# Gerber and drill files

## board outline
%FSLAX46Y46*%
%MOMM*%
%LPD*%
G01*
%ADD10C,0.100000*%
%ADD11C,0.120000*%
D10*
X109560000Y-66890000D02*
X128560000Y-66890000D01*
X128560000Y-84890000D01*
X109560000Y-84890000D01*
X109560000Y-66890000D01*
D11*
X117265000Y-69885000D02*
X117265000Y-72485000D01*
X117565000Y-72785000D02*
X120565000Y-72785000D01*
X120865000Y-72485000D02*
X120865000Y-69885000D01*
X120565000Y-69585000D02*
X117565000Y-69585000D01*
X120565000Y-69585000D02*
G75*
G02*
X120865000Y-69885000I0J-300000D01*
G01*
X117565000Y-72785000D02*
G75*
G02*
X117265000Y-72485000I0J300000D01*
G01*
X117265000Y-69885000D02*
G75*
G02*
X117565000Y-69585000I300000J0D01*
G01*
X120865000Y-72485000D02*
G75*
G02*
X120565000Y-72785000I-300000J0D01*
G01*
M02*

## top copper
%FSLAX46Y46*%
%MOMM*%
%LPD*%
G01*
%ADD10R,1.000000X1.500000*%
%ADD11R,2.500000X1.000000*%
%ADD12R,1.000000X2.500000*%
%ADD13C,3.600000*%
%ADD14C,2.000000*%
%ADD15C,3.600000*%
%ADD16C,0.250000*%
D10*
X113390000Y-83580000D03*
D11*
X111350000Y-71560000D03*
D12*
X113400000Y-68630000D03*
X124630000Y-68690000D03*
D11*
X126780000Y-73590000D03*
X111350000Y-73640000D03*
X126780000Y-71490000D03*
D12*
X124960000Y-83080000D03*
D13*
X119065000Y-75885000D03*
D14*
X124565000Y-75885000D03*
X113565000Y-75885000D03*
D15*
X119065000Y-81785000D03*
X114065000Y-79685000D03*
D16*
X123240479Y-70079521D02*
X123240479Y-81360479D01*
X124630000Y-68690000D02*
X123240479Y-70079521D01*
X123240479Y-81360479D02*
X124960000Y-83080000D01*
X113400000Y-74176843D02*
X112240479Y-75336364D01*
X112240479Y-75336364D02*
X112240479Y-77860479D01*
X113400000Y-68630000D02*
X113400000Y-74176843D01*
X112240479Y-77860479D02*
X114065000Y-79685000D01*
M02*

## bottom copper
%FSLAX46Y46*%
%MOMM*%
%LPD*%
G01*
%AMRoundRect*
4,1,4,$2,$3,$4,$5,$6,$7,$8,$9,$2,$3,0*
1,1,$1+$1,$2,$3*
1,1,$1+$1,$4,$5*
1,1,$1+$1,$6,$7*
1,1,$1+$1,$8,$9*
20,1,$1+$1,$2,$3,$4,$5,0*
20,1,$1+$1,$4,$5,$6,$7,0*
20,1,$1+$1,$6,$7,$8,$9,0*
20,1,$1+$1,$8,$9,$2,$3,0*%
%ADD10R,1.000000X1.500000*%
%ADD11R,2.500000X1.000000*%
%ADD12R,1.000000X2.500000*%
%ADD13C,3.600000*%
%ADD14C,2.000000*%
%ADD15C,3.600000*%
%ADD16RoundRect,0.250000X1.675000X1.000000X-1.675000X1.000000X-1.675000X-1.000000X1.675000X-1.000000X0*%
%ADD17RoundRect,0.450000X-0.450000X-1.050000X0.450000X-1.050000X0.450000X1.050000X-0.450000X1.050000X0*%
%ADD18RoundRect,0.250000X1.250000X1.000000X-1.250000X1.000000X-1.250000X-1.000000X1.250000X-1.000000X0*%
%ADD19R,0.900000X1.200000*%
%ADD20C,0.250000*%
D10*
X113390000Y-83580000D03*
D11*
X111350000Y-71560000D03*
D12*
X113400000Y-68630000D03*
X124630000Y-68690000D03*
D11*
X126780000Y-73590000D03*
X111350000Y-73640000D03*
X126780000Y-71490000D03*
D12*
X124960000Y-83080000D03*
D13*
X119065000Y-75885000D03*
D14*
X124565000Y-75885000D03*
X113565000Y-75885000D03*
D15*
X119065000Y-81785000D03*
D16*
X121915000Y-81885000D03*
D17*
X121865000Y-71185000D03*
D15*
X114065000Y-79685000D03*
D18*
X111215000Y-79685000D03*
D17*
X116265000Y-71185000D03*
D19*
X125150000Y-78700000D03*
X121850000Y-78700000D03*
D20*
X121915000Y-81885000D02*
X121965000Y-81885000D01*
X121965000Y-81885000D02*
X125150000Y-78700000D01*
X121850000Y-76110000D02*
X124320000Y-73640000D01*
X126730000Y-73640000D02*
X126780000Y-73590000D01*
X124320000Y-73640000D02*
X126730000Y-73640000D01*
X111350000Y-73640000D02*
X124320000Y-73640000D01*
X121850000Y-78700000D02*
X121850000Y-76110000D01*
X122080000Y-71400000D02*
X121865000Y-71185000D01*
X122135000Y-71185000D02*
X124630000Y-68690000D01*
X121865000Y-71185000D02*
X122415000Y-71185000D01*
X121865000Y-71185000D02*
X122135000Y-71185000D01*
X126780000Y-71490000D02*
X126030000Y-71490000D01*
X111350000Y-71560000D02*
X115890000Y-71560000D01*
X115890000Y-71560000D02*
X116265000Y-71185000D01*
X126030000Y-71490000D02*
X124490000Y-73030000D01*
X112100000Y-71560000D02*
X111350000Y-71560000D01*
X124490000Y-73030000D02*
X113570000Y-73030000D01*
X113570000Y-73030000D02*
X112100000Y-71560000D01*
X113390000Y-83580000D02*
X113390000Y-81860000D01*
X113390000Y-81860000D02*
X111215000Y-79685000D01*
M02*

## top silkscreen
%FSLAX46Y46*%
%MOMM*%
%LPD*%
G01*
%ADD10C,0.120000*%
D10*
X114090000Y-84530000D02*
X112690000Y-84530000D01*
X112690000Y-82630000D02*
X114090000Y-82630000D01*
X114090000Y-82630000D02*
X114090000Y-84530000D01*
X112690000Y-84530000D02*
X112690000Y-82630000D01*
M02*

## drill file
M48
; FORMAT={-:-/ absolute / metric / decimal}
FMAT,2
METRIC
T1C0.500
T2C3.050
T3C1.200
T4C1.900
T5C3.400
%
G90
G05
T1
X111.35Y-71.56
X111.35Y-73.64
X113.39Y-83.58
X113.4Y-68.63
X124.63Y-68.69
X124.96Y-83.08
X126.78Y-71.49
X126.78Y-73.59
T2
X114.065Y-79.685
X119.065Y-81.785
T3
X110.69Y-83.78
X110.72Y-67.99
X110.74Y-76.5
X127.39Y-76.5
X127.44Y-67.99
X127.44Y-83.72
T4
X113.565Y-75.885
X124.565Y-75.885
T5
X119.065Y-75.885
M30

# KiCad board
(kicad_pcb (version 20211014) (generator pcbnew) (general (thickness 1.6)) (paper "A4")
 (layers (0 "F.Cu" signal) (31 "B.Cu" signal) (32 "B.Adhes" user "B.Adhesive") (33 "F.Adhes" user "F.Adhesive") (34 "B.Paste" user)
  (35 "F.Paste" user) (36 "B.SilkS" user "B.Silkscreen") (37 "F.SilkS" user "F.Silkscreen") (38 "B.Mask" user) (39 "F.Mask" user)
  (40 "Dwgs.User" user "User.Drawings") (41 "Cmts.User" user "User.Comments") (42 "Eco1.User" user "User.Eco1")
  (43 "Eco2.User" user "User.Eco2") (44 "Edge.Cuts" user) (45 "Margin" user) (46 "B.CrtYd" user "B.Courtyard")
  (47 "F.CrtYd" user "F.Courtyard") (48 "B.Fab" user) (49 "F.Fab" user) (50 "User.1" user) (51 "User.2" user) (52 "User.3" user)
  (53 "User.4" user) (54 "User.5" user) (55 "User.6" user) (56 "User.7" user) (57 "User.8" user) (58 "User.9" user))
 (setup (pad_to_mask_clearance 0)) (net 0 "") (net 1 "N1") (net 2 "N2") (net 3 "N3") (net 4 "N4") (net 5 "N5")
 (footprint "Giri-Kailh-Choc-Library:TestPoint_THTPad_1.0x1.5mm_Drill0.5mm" (layer "F.Cu") (at 113.39 83.58 -90)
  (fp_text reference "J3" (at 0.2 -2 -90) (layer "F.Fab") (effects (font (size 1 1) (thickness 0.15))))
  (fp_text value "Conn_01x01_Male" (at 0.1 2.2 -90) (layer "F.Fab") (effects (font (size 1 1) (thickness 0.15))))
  (fp_line (start 0.95 -0.7) (end 0.95 0.7) (layer "F.SilkS") (width 0.12))
  (fp_line (start -0.95 0.7) (end -0.95 -0.7) (layer "F.SilkS") (width 0.12))
  (fp_line (start -0.95 -0.7) (end 0.95 -0.7) (layer "F.SilkS") (width 0.12))
  (fp_line (start 0.95 0.7) (end -0.95 0.7) (layer "F.SilkS") (width 0.12))
  (pad "1" thru_hole rect (at 0 0 270) (size 1.5 1) (drill 0.5) (layers *.Cu *.Mask) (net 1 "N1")))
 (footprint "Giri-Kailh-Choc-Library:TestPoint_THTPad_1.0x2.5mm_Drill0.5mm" (layer "F.Cu") (at 111.35 71.56)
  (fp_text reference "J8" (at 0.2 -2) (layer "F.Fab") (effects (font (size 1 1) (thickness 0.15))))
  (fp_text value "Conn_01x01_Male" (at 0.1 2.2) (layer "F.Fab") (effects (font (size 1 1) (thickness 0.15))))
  (pad "1" thru_hole rect (at 0 0) (size 2.5 1) (drill 0.5) (layers *.Cu *.Mask) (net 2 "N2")))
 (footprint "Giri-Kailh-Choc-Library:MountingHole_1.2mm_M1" (layer "F.Cu") (at 110.69 83.78)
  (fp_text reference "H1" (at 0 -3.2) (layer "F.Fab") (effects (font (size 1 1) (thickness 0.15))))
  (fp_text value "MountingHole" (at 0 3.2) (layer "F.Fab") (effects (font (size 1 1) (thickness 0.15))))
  (pad "" np_thru_hole circle (at 0 0) (size 1.2 1.2) (drill 1.2) (layers F&B.Cu *.Mask)))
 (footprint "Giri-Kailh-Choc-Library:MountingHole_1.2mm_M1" (layer "F.Cu") (at 127.39 76.5)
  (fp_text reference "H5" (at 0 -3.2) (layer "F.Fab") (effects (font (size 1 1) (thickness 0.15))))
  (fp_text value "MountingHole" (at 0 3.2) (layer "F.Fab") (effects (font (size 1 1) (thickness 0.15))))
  (pad "" np_thru_hole circle (at 0 0) (size 1.2 1.2) (drill 1.2) (layers F&B.Cu *.Mask)))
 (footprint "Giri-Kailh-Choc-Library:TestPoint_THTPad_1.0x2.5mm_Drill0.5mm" (layer "F.Cu") (at 113.4 68.63 90)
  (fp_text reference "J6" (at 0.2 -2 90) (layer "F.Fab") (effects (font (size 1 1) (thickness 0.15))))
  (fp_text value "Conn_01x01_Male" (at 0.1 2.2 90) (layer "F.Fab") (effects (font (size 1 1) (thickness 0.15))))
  (pad "1" thru_hole rect (at 0 0 90) (size 2.5 1) (drill 0.5) (layers *.Cu *.Mask) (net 1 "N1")))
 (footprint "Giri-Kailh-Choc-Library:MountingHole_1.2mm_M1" (layer "F.Cu") (at 127.44 83.72)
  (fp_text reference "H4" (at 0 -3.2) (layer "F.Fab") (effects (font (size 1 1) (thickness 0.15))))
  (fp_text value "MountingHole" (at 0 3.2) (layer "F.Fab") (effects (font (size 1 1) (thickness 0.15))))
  (pad "" np_thru_hole circle (at 0 0) (size 1.2 1.2) (drill 1.2) (layers F&B.Cu *.Mask)))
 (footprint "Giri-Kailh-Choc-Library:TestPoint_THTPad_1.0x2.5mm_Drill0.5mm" (layer "F.Cu") (at 124.63 68.69 90)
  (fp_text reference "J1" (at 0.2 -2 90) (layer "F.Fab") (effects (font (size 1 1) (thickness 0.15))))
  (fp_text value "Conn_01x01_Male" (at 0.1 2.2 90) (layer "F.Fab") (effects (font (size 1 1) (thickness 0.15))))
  (pad "1" thru_hole rect (at 0 0 90) (size 2.5 1) (drill 0.5) (layers *.Cu *.Mask) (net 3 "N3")))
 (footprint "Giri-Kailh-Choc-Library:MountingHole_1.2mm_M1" (layer "F.Cu") (at 127.44 67.99)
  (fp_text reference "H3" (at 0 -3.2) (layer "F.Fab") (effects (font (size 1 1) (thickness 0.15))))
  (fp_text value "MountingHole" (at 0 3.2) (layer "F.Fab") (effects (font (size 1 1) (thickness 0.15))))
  (pad "" np_thru_hole circle (at 0 0) (size 1.2 1.2) (drill 1.2) (layers F&B.Cu *.Mask)))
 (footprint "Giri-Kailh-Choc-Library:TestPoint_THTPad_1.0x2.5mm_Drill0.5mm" (layer "F.Cu") (at 126.78 73.59)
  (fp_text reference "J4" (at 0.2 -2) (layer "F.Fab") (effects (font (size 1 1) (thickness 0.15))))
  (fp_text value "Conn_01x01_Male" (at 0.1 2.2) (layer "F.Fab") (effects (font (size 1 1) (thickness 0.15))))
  (pad "1" thru_hole rect (at 0 0) (size 2.5 1) (drill 0.5) (layers *.Cu *.Mask) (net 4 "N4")))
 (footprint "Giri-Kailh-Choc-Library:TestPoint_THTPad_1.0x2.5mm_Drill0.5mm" (layer "F.Cu") (at 111.35 73.64)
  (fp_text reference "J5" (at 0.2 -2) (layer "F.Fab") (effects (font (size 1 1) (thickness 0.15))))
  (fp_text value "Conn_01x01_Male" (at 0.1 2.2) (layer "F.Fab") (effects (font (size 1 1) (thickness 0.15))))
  (pad "1" thru_hole rect (at 0 0) (size 2.5 1) (drill 0.5) (layers *.Cu *.Mask) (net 4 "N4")))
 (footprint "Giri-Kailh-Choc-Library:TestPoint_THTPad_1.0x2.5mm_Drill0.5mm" (layer "F.Cu") (at 126.78 71.49)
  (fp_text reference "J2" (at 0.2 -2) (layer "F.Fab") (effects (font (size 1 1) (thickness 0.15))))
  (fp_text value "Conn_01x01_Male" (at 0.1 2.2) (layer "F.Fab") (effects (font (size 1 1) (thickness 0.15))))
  (pad "1" thru_hole rect (at 0 0) (size 2.5 1) (drill 0.5) (layers *.Cu *.Mask) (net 2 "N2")))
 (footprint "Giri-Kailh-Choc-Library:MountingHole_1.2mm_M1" (layer "F.Cu") (at 110.74 76.5)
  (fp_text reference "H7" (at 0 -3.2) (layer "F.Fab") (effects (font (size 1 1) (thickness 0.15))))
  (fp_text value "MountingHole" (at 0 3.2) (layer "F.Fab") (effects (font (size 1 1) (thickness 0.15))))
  (pad "" np_thru_hole circle (at 0 0) (size 1.2 1.2) (drill 1.2) (layers F&B.Cu *.Mask)))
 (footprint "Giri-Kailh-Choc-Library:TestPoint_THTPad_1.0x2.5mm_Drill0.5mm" (layer "F.Cu") (at 124.96 83.08 90)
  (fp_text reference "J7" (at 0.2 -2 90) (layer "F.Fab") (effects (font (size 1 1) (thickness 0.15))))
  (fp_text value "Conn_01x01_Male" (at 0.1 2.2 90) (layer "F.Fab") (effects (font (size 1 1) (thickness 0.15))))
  (pad "1" thru_hole rect (at 0 0 90) (size 2.5 1) (drill 0.5) (layers *.Cu *.Mask) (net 3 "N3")))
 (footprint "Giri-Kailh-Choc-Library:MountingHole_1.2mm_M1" (layer "F.Cu") (at 110.72 67.99)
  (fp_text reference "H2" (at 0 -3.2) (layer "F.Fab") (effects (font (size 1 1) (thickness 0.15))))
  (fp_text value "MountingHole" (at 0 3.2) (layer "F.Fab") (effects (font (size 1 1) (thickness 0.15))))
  (pad "" np_thru_hole circle (at 0 0) (size 1.2 1.2) (drill 1.2) (layers F&B.Cu *.Mask)))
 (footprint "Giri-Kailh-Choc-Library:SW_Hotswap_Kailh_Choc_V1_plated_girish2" (layer "F.Cu") (at 119.065 75.885)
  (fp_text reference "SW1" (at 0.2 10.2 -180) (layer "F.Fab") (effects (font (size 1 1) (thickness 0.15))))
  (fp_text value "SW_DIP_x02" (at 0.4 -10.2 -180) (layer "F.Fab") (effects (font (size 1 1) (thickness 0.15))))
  (fp_line (start -1.8 -6) (end -1.8 -3.4) (layer "Edge.Cuts") (width 0.12))
  (fp_line (start -1.5 -3.1) (end 1.5 -3.1) (layer "Edge.Cuts") (width 0.12))
  (fp_line (start 1.8 -3.4) (end 1.8 -6) (layer "Edge.Cuts") (width 0.12))
  (fp_line (start 1.5 -6.3) (end -1.5 -6.3) (layer "Edge.Cuts") (width 0.12))
  (fp_arc (start 1.5 -6.3) (mid 1.712132 -6.212132) (end 1.8 -6) (layer "Edge.Cuts") (width 0.12))
  (fp_arc (start -1.5 -3.1) (mid -1.712132 -3.187868) (end -1.8 -3.4) (layer "Edge.Cuts") (width 0.12))
  (fp_arc (start -1.8 -6) (mid -1.712132 -6.212132) (end -1.5 -6.3) (layer "Edge.Cuts") (width 0.12))
  (fp_arc (start 1.8 -3.4) (mid 1.712132 -3.187868) (end 1.5 -3.1) (layer "Edge.Cuts") (width 0.12))
  (pad "" np_thru_hole circle (at 0 0 180) (size 3.6 3.6) (drill 3.4) (layers F&B.Cu *.Mask))
  (pad "" smd roundrect (at 3.5 6 180) (size 2.55 2.5) (layers "B.Paste" "B.Mask") (roundrect_rratio 0.1))
  (pad "" np_thru_hole circle (at 5.5 0 180) (size 2 2) (drill 1.9) (layers F&B.Cu *.Mask))
  (pad "" np_thru_hole circle (at -5.5 0 180) (size 2 2) (drill 1.9) (layers F&B.Cu *.Mask))
  (pad "" smd roundrect (at -8.5 3.8 180) (size 1.9 2.5) (layers "B.Paste" "B.Mask") (roundrect_rratio 0.1))
  (pad "1" thru_hole circle (at 0 5.9 180) (size 3.6 3.6) (drill 3.05) (layers *.Cu "B.Mask") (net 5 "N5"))
  (pad "1" smd roundrect (at 2.85 6 180) (size 3.85 2.5) (layers "B.Cu" "B.Paste" "B.Mask") (roundrect_rratio 0.1) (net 5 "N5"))
  (pad "2" smd roundrect (at 2.8 -4.7) (size 1.8 3) (layers "B.Cu" "B.Paste" "B.Mask") (roundrect_rratio 0.25) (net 3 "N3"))
  (pad "3" thru_hole circle (at -5 3.8 180) (size 3.6 3.6) (drill 3.05) (layers *.Cu "B.Mask") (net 1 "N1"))
  (pad "3" smd roundrect (at -7.85 3.8 180) (size 3 2.5) (layers "B.Cu" "B.Paste" "B.Mask") (roundrect_rratio 0.1) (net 1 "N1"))
  (pad "4" smd roundrect (at -2.8 -4.7) (size 1.8 3) (layers "B.Cu" "B.Paste" "B.Mask") (roundrect_rratio 0.25) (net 2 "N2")))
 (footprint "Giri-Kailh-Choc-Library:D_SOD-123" (layer "B.Cu") (at 123.5 78.7 180)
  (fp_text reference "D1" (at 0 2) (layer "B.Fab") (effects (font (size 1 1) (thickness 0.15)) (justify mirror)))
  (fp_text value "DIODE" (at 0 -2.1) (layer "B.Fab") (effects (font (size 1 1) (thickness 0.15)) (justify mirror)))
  (pad "1" smd rect (at -1.65 0 180) (size 0.9 1.2) (layers "B.Cu" "B.Paste" "B.Mask") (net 5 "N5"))
  (pad "2" smd rect (at 1.65 0 180) (size 0.9 1.2) (layers "B.Cu" "B.Paste" "B.Mask") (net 4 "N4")))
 (gr_rect (start 109.56 84.89) (end 128.56 66.89) (layer "Edge.Cuts") (width 0.1) (fill none))
 (segment (start 121.915 81.885) (end 121.965 81.885) (width 0.25) (layer "B.Cu") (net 5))
 (segment (start 121.965 81.885) (end 125.15 78.7) (width 0.25) (layer "B.Cu") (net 5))
 (segment (start 121.85 76.11) (end 124.32 73.64) (width 0.25) (layer "B.Cu") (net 4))
 (segment (start 126.73 73.64) (end 126.78 73.59) (width 0.25) (layer "B.Cu") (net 4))
 (segment (start 124.32 73.64) (end 126.73 73.64) (width 0.25) (layer "B.Cu") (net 4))
 (segment (start 111.35 73.64) (end 124.32 73.64) (width 0.25) (layer "B.Cu") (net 4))
 (segment (start 121.85 78.7) (end 121.85 76.11) (width 0.25) (layer "B.Cu") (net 4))
 (segment (start 123.240479 70.079521) (end 123.240479 81.360479) (width 0.25) (layer "F.Cu") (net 3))
 (segment (start 124.63 68.69) (end 123.240479 70.079521) (width 0.25) (layer "F.Cu") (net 3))
 (segment (start 123.240479 81.360479) (end 124.96 83.08) (width 0.25) (layer "F.Cu") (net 3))
 (segment (start 122.08 71.4) (end 121.865 71.185) (width 0.25) (layer "B.Cu") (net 3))
 (segment (start 122.135 71.185) (end 124.63 68.69) (width 0.25) (layer "B.Cu") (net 3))
 (segment (start 121.865 71.185) (end 122.415 71.185) (width 0.25) (layer "B.Cu") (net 3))
 (segment (start 121.865 71.185) (end 122.135 71.185) (width 0.25) (layer "B.Cu") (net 3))
 (segment (start 126.78 71.49) (end 126.03 71.49) (width 0.25) (layer "B.Cu") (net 2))
 (segment (start 111.35 71.56) (end 115.89 71.56) (width 0.25) (layer "B.Cu") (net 2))
 (segment (start 115.89 71.56) (end 116.265 71.185) (width 0.25) (layer "B.Cu") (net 2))
 (segment (start 126.03 71.49) (end 124.49 73.03) (width 0.25) (layer "B.Cu") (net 2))
 (segment (start 112.1 71.56) (end 111.35 71.56) (width 0.25) (layer "B.Cu") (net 2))
 (segment (start 124.49 73.03) (end 113.57 73.03) (width 0.25) (layer "B.Cu") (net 2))
 (segment (start 113.57 73.03) (end 112.1 71.56) (width 0.25) (layer "B.Cu") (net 2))
 (segment (start 113.4 74.176843) (end 112.240479 75.336364) (width 0.25) (layer "F.Cu") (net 1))
 (segment (start 112.240479 75.336364) (end 112.240479 77.860479) (width 0.25) (layer "F.Cu") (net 1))
 (segment (start 113.4 68.63) (end 113.4 74.176843) (width 0.25) (layer "F.Cu") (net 1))
 (segment (start 112.240479 77.860479) (end 114.065 79.685) (width 0.25) (layer "F.Cu") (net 1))
 (segment (start 113.39 83.58) (end 113.39 81.86) (width 0.25) (layer "B.Cu") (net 1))
 (segment (start 113.39 81.86) (end 111.215 79.685) (width 0.25) (layer "B.Cu") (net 1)))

